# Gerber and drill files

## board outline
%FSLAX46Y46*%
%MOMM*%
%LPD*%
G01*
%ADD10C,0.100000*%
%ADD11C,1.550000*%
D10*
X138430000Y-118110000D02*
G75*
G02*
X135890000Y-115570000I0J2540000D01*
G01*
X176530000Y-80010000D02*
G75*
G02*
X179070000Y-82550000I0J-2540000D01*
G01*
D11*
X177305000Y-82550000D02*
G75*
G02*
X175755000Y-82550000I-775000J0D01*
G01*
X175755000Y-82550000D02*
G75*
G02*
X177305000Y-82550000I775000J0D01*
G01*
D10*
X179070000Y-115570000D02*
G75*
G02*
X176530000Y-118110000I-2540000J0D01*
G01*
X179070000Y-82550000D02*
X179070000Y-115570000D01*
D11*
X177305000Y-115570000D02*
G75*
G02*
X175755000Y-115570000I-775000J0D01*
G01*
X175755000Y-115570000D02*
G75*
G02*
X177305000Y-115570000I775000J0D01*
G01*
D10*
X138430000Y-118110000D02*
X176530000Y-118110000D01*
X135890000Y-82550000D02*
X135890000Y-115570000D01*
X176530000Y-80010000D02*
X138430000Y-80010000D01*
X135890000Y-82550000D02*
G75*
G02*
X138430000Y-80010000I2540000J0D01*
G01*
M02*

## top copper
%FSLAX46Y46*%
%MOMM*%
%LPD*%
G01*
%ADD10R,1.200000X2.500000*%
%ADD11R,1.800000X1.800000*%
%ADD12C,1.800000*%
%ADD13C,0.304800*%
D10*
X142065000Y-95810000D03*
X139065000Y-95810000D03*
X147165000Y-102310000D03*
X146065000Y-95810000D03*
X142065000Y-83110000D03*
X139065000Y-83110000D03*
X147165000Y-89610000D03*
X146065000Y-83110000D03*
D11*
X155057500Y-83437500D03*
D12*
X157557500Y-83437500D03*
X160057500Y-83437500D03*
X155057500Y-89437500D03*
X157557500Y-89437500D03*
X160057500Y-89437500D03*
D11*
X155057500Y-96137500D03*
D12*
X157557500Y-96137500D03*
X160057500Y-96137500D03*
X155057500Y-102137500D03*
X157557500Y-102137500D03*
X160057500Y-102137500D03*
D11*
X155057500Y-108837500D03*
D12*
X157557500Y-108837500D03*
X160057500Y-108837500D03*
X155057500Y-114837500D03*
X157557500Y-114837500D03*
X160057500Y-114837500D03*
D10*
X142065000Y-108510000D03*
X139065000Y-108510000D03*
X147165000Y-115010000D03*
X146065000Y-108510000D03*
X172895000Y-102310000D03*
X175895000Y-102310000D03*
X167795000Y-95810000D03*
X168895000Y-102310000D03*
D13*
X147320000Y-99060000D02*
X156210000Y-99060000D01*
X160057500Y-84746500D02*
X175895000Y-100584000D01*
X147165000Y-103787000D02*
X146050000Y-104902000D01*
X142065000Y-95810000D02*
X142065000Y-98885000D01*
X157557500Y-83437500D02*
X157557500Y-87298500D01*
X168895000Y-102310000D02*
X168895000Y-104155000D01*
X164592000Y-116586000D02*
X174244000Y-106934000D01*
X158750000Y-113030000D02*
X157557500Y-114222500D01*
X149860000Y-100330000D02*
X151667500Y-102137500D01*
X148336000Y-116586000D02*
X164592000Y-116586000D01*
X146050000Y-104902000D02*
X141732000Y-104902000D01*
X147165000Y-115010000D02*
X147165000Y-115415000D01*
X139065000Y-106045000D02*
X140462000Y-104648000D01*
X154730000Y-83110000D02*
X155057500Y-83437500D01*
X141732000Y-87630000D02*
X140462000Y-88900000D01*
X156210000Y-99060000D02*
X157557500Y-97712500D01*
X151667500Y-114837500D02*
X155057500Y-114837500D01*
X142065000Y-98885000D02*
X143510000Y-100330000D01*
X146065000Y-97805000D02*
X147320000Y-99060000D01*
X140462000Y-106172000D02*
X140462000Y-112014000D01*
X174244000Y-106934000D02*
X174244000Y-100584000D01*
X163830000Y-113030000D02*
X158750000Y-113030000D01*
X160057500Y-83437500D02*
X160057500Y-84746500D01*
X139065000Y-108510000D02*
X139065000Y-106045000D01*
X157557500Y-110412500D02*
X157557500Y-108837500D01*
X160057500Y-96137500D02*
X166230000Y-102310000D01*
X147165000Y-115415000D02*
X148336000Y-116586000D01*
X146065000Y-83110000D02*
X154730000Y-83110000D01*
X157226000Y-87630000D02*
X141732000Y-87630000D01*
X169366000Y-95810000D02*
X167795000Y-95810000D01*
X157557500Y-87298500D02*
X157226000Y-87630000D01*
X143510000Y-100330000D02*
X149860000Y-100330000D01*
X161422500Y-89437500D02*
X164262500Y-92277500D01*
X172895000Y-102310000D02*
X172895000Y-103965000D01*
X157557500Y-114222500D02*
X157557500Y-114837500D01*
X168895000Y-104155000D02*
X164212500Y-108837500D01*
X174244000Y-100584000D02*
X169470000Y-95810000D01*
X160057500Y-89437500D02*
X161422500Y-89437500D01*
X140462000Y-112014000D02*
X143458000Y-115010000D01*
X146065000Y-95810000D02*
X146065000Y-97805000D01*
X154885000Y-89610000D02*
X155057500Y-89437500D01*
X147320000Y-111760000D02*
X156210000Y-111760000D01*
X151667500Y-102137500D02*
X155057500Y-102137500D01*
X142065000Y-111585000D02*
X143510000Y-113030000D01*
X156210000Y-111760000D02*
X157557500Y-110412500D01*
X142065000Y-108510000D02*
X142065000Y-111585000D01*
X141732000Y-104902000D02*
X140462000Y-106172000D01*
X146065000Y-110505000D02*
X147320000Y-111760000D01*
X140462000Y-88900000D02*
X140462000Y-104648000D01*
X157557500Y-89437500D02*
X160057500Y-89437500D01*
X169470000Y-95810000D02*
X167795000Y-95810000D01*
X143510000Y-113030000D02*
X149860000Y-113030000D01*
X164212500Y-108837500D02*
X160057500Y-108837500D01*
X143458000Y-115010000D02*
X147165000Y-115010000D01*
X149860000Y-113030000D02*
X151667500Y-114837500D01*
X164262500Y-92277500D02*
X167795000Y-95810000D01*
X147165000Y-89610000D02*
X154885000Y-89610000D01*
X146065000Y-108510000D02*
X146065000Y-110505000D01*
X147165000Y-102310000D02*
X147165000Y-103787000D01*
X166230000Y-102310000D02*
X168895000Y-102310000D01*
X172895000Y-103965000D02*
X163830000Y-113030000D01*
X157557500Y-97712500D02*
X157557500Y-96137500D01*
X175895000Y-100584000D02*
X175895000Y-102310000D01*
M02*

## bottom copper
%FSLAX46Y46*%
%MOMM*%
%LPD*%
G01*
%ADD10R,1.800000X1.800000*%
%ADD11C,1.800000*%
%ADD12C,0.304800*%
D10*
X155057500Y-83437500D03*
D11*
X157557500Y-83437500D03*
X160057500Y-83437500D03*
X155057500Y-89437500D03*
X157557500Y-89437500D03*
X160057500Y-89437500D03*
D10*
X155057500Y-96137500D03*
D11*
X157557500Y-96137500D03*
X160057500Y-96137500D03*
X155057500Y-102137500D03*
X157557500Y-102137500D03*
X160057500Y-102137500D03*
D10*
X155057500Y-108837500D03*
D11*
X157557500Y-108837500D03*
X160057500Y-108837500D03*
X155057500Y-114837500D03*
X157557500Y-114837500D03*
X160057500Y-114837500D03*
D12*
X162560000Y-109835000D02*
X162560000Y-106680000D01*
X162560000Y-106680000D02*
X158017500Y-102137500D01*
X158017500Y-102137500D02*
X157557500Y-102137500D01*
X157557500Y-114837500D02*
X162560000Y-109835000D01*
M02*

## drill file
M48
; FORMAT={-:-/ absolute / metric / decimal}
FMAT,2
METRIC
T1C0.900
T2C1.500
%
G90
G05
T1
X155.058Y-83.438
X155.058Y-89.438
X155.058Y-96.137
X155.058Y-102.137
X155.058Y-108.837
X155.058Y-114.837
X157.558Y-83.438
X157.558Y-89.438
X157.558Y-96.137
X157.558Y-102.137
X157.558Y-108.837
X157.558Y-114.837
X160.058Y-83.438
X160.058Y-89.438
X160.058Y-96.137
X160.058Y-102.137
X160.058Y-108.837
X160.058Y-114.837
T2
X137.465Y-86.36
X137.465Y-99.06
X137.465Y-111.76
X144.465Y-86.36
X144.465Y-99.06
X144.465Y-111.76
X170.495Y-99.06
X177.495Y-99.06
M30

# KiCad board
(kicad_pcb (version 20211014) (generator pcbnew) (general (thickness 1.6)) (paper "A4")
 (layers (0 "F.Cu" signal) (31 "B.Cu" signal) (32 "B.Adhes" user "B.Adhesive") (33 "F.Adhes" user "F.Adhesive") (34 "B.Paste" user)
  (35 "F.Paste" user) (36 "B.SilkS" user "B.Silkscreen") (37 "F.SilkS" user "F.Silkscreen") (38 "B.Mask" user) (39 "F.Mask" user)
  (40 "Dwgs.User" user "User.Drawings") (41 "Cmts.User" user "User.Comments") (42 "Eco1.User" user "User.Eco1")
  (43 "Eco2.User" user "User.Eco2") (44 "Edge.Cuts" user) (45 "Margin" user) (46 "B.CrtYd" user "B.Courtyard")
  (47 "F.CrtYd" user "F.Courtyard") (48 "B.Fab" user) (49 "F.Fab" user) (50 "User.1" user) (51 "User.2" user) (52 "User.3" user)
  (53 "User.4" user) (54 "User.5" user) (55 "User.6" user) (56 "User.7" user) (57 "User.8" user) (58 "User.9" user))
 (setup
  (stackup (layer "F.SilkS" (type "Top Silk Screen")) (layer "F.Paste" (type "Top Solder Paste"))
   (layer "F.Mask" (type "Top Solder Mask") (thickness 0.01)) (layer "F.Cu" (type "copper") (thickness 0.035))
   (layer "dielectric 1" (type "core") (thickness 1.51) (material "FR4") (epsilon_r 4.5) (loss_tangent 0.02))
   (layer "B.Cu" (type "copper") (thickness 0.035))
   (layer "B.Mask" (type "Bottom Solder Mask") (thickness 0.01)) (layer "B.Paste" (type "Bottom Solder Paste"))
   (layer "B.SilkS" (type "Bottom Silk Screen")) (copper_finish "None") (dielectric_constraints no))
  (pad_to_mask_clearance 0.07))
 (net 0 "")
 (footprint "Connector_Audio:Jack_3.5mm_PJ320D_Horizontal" (layer "F.Cu") (at 142.24 99.06)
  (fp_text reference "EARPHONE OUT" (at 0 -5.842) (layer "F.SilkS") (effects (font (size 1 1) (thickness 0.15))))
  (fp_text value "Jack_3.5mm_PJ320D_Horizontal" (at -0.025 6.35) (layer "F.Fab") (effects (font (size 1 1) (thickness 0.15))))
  (pad "" np_thru_hole circle (at -4.775 0) (size 1.5 1.5) (drill 1.5) (layers *.Cu *.Mask))
  (pad "" np_thru_hole circle (at 2.225 0) (size 1.5 1.5) (drill 1.5) (layers *.Cu *.Mask))
  (pad "R1" smd rect (at -0.175 -3.25) (size 1.2 2.5) (layers "F.Cu" "F.Paste" "F.Mask"))
  (pad "R2" smd rect (at -3.175 -3.25) (size 1.2 2.5) (layers "F.Cu" "F.Paste" "F.Mask"))
  (pad "S" smd rect (at 4.925 3.25) (size 1.2 2.5) (layers "F.Cu" "F.Paste" "F.Mask"))
  (pad "T" smd rect (at 3.825 -3.25) (size 1.2 2.5) (layers "F.Cu" "F.Paste" "F.Mask")))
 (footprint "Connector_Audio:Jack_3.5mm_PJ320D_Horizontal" (layer "F.Cu") (at 142.24 86.36)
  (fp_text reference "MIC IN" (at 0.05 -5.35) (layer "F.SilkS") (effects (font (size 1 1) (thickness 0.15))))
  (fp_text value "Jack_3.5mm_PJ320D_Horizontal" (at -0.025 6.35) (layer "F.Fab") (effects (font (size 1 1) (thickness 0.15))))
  (pad "" np_thru_hole circle (at 2.225 0) (size 1.5 1.5) (drill 1.5) (layers *.Cu *.Mask))
  (pad "" np_thru_hole circle (at -4.775 0) (size 1.5 1.5) (drill 1.5) (layers *.Cu *.Mask))
  (pad "R1" smd rect (at -0.175 -3.25) (size 1.2 2.5) (layers "F.Cu" "F.Paste" "F.Mask"))
  (pad "R2" smd rect (at -3.175 -3.25) (size 1.2 2.5) (layers "F.Cu" "F.Paste" "F.Mask"))
  (pad "S" smd rect (at 4.925 3.25) (size 1.2 2.5) (layers "F.Cu" "F.Paste" "F.Mask"))
  (pad "T" smd rect (at 3.825 -3.25) (size 1.2 2.5) (layers "F.Cu" "F.Paste" "F.Mask")))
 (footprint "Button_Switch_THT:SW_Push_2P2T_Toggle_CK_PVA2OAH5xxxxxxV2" (layer "F.Cu") (at 155.0575 83.4375)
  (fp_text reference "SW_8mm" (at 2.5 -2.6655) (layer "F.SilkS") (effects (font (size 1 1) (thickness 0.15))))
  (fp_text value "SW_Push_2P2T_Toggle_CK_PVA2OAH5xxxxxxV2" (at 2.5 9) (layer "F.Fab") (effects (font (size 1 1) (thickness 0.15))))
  (pad "1" thru_hole rect (at 0 0) (size 1.8 1.8) (drill 0.9) (layers *.Cu *.Mask))
  (pad "2" thru_hole circle (at 2.5 0) (size 1.8 1.8) (drill 0.9) (layers *.Cu *.Mask))
  (pad "3" thru_hole circle (at 5 0) (size 1.8 1.8) (drill 0.9) (layers *.Cu *.Mask))
  (pad "4" thru_hole circle (at 0 6) (size 1.8 1.8) (drill 0.9) (layers *.Cu *.Mask))
  (pad "5" thru_hole circle (at 2.5 6) (size 1.8 1.8) (drill 0.9) (layers *.Cu *.Mask))
  (pad "6" thru_hole circle (at 5 6) (size 1.8 1.8) (drill 0.9) (layers *.Cu *.Mask)))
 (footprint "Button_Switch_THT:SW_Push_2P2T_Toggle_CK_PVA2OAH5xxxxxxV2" (layer "F.Cu") (at 155.0575 96.1375)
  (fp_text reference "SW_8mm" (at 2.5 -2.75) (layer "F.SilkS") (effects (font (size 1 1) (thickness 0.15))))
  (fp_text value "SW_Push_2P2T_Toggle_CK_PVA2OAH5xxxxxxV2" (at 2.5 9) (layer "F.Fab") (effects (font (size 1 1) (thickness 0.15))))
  (pad "1" thru_hole rect (at 0 0) (size 1.8 1.8) (drill 0.9) (layers *.Cu *.Mask))
  (pad "2" thru_hole circle (at 2.5 0) (size 1.8 1.8) (drill 0.9) (layers *.Cu *.Mask))
  (pad "3" thru_hole circle (at 5 0) (size 1.8 1.8) (drill 0.9) (layers *.Cu *.Mask))
  (pad "4" thru_hole circle (at 0 6) (size 1.8 1.8) (drill 0.9) (layers *.Cu *.Mask))
  (pad "5" thru_hole circle (at 2.5 6) (size 1.8 1.8) (drill 0.9) (layers *.Cu *.Mask))
  (pad "6" thru_hole circle (at 5 6) (size 1.8 1.8) (drill 0.9) (layers *.Cu *.Mask)))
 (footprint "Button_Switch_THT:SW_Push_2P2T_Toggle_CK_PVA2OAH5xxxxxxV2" (layer "F.Cu") (at 155.0575 108.8375)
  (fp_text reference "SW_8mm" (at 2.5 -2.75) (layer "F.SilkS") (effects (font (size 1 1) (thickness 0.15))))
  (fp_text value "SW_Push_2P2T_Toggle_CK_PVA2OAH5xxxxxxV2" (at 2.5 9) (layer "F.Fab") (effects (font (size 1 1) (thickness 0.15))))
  (pad "1" thru_hole rect (at 0 0) (size 1.8 1.8) (drill 0.9) (layers *.Cu *.Mask))
  (pad "2" thru_hole circle (at 2.5 0) (size 1.8 1.8) (drill 0.9) (layers *.Cu *.Mask))
  (pad "3" thru_hole circle (at 5 0) (size 1.8 1.8) (drill 0.9) (layers *.Cu *.Mask))
  (pad "4" thru_hole circle (at 0 6) (size 1.8 1.8) (drill 0.9) (layers *.Cu *.Mask))
  (pad "5" thru_hole circle (at 2.5 6) (size 1.8 1.8) (drill 0.9) (layers *.Cu *.Mask))
  (pad "6" thru_hole circle (at 5 6) (size 1.8 1.8) (drill 0.9) (layers *.Cu *.Mask)))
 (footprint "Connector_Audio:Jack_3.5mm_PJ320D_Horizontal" (layer "F.Cu") (at 142.24 111.76)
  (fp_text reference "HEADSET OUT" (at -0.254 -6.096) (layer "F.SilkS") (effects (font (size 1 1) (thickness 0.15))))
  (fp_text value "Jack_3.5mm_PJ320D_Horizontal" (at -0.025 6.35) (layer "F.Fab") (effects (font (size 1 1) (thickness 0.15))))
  (pad "" np_thru_hole circle (at -4.775 0) (size 1.5 1.5) (drill 1.5) (layers *.Cu *.Mask))
  (pad "" np_thru_hole circle (at 2.225 0) (size 1.5 1.5) (drill 1.5) (layers *.Cu *.Mask))
  (pad "R1" smd rect (at -0.175 -3.25) (size 1.2 2.5) (layers "F.Cu" "F.Paste" "F.Mask"))
  (pad "R2" smd rect (at -3.175 -3.25) (size 1.2 2.5) (layers "F.Cu" "F.Paste" "F.Mask"))
  (pad "S" smd rect (at 4.925 3.25) (size 1.2 2.5) (layers "F.Cu" "F.Paste" "F.Mask"))
  (pad "T" smd rect (at 3.825 -3.25) (size 1.2 2.5) (layers "F.Cu" "F.Paste" "F.Mask")))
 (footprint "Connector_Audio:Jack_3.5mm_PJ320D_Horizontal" (layer "F.Cu") (at 172.72 99.06 180)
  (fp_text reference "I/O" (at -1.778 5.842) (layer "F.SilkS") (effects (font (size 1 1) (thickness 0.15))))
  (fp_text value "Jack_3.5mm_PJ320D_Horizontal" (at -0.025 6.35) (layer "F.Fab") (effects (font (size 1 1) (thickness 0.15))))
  (pad "" np_thru_hole circle (at -4.775 0 180) (size 1.5 1.5) (drill 1.5) (layers *.Cu *.Mask))
  (pad "" np_thru_hole circle (at 2.225 0 180) (size 1.5 1.5) (drill 1.5) (layers *.Cu *.Mask))
  (pad "R1" smd rect (at -0.175 -3.25 180) (size 1.2 2.5) (layers "F.Cu" "F.Paste" "F.Mask"))
  (pad "R2" smd rect (at -3.175 -3.25 180) (size 1.2 2.5) (layers "F.Cu" "F.Paste" "F.Mask"))
  (pad "S" smd rect (at 4.925 3.25 180) (size 1.2 2.5) (layers "F.Cu" "F.Paste" "F.Mask"))
  (pad "T" smd rect (at 3.825 -3.25 180) (size 1.2 2.5) (layers "F.Cu" "F.Paste" "F.Mask")))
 (gr_arc (start 138.43 118.11) (mid 136.633949 117.366051) (end 135.89 115.57) (layer "Edge.Cuts") (width 0.1))
 (gr_arc (start 176.53 80.01) (mid 178.326051 80.753949) (end 179.07 82.55) (layer "Edge.Cuts") (width 0.1))
 (gr_circle (center 176.53 82.55) (end 178.03 82.55) (layer "Edge.Cuts") (width 0.1) (fill solid))
 (gr_arc (start 179.07 115.57) (mid 178.326051 117.366051) (end 176.53 118.11) (layer "Edge.Cuts") (width 0.1))
 (gr_line (start 179.07 82.55) (end 179.07 115.57) (layer "Edge.Cuts") (width 0.1))
 (gr_circle (center 176.53 115.57) (end 178.03 115.57) (layer "Edge.Cuts") (width 0.1) (fill solid))
 (gr_line (start 138.43 118.11) (end 176.53 118.11) (layer "Edge.Cuts") (width 0.1))
 (gr_line (start 135.89 82.55) (end 135.89 115.57) (layer "Edge.Cuts") (width 0.1))
 (gr_line (start 176.53 80.01) (end 138.43 80.01) (layer "Edge.Cuts") (width 0.1))
 (gr_arc (start 135.89 82.55) (mid 136.633949 80.753949) (end 138.43 80.01) (layer "Edge.Cuts") (width 0.1))
 (segment (start 147.32 99.06) (end 156.21 99.06) (width 0.3048) (layer "F.Cu") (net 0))
 (segment (start 160.0575 84.7465) (end 175.895 100.584) (width 0.3048) (layer "F.Cu") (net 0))
 (segment (start 147.165 103.787) (end 146.05 104.902) (width 0.3048) (layer "F.Cu") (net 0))
 (segment (start 142.065 95.81) (end 142.065 98.885) (width 0.3048) (layer "F.Cu") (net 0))
 (segment (start 157.5575 83.4375) (end 157.5575 87.2985) (width 0.3048) (layer "F.Cu") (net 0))
 (segment (start 168.895 102.31) (end 168.895 104.155) (width 0.3048) (layer "F.Cu") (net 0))
 (segment (start 164.592 116.586) (end 174.244 106.934) (width 0.3048) (layer "F.Cu") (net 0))
 (segment (start 158.75 113.03) (end 157.5575 114.2225) (width 0.3048) (layer "F.Cu") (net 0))
 (segment (start 149.86 100.33) (end 151.6675 102.1375) (width 0.3048) (layer "F.Cu") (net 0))
 (segment (start 148.336 116.586) (end 164.592 116.586) (width 0.3048) (layer "F.Cu") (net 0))
 (segment (start 146.05 104.902) (end 141.732 104.902) (width 0.3048) (layer "F.Cu") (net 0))
 (segment (start 147.165 115.01) (end 147.165 115.415) (width 0.3048) (layer "F.Cu") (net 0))
 (segment (start 139.065 106.045) (end 140.462 104.648) (width 0.3048) (layer "F.Cu") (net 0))
 (segment (start 154.73 83.11) (end 155.0575 83.4375) (width 0.3048) (layer "F.Cu") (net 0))
 (segment (start 141.732 87.63) (end 140.462 88.9) (width 0.3048) (layer "F.Cu") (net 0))
 (segment (start 156.21 99.06) (end 157.5575 97.7125) (width 0.3048) (layer "F.Cu") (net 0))
 (segment (start 151.6675 114.8375) (end 155.0575 114.8375) (width 0.3048) (layer "F.Cu") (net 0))
 (segment (start 142.065 98.885) (end 143.51 100.33) (width 0.3048) (layer "F.Cu") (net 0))
 (segment (start 146.065 97.805) (end 147.32 99.06) (width 0.3048) (layer "F.Cu") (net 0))
 (segment (start 140.462 106.172) (end 140.462 112.014) (width 0.3048) (layer "F.Cu") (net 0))
 (segment (start 174.244 106.934) (end 174.244 100.584) (width 0.3048) (layer "F.Cu") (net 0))
 (segment (start 163.83 113.03) (end 158.75 113.03) (width 0.3048) (layer "F.Cu") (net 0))
 (segment (start 160.0575 83.4375) (end 160.0575 84.7465) (width 0.3048) (layer "F.Cu") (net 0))
 (segment (start 139.065 108.51) (end 139.065 106.045) (width 0.3048) (layer "F.Cu") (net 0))
 (segment (start 157.5575 110.4125) (end 157.5575 108.8375) (width 0.3048) (layer "F.Cu") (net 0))
 (segment (start 160.0575 96.1375) (end 166.23 102.31) (width 0.3048) (layer "F.Cu") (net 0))
 (segment (start 147.165 115.415) (end 148.336 116.586) (width 0.3048) (layer "F.Cu") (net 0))
 (segment (start 146.065 83.11) (end 154.73 83.11) (width 0.3048) (layer "F.Cu") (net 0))
 (segment (start 157.226 87.63) (end 141.732 87.63) (width 0.3048) (layer "F.Cu") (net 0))
 (segment (start 169.366 95.81) (end 167.795 95.81) (width 0.3048) (layer "F.Cu") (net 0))
 (segment (start 157.5575 87.2985) (end 157.226 87.63) (width 0.3048) (layer "F.Cu") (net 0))
 (segment (start 143.51 100.33) (end 149.86 100.33) (width 0.3048) (layer "F.Cu") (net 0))
 (segment (start 161.4225 89.4375) (end 164.2625 92.2775) (width 0.3048) (layer "F.Cu") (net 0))
 (segment (start 172.895 102.31) (end 172.895 103.965) (width 0.3048) (layer "F.Cu") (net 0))
 (segment (start 157.5575 114.2225) (end 157.5575 114.8375) (width 0.3048) (layer "F.Cu") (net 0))
 (segment (start 168.895 104.155) (end 164.2125 108.8375) (width 0.3048) (layer "F.Cu") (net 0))
 (segment (start 174.244 100.584) (end 169.47 95.81) (width 0.3048) (layer "F.Cu") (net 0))
 (segment (start 160.0575 89.4375) (end 161.4225 89.4375) (width 0.3048) (layer "F.Cu") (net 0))
 (segment (start 140.462 112.014) (end 143.458 115.01) (width 0.3048) (layer "F.Cu") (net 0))
 (segment (start 146.065 95.81) (end 146.065 97.805) (width 0.3048) (layer "F.Cu") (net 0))
 (segment (start 154.885 89.61) (end 155.0575 89.4375) (width 0.3048) (layer "F.Cu") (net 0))
 (segment (start 147.32 111.76) (end 156.21 111.76) (width 0.3048) (layer "F.Cu") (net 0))
 (segment (start 151.6675 102.1375) (end 155.0575 102.1375) (width 0.3048) (layer "F.Cu") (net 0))
 (segment (start 142.065 111.585) (end 143.51 113.03) (width 0.3048) (layer "F.Cu") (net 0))
 (segment (start 156.21 111.76) (end 157.5575 110.4125) (width 0.3048) (layer "F.Cu") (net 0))
 (segment (start 142.065 108.51) (end 142.065 111.585) (width 0.3048) (layer "F.Cu") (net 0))
 (segment (start 141.732 104.902) (end 140.462 106.172) (width 0.3048) (layer "F.Cu") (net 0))
 (segment (start 146.065 110.505) (end 147.32 111.76) (width 0.3048) (layer "F.Cu") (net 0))
 (segment (start 140.462 88.9) (end 140.462 104.648) (width 0.3048) (layer "F.Cu") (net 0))
 (segment (start 157.5575 89.4375) (end 160.0575 89.4375) (width 0.3048) (layer "F.Cu") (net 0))
 (segment (start 169.47 95.81) (end 167.795 95.81) (width 0.3048) (layer "F.Cu") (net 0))
 (segment (start 143.51 113.03) (end 149.86 113.03) (width 0.3048) (layer "F.Cu") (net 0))
 (segment (start 164.2125 108.8375) (end 160.0575 108.8375) (width 0.3048) (layer "F.Cu") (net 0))
 (segment (start 143.458 115.01) (end 147.165 115.01) (width 0.3048) (layer "F.Cu") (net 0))
 (segment (start 149.86 113.03) (end 151.6675 114.8375) (width 0.3048) (layer "F.Cu") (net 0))
 (segment (start 164.2625 92.2775) (end 167.795 95.81) (width 0.3048) (layer "F.Cu") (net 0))
 (segment (start 147.165 89.61) (end 154.885 89.61) (width 0.3048) (layer "F.Cu") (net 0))
 (segment (start 146.065 108.51) (end 146.065 110.505) (width 0.3048) (layer "F.Cu") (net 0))
 (segment (start 147.165 102.31) (end 147.165 103.787) (width 0.3048) (layer "F.Cu") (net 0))
 (segment (start 166.23 102.31) (end 168.895 102.31) (width 0.3048) (layer "F.Cu") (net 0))
 (segment (start 172.895 103.965) (end 163.83 113.03) (width 0.3048) (layer "F.Cu") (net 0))
 (segment (start 157.5575 97.7125) (end 157.5575 96.1375) (width 0.3048) (layer "F.Cu") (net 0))
 (segment (start 175.895 100.584) (end 175.895 102.31) (width 0.3048) (layer "F.Cu") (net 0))
 (segment (start 162.56 109.835) (end 162.56 106.68) (width 0.3048) (layer "B.Cu") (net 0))
 (segment (start 162.56 106.68) (end 158.0175 102.1375) (width 0.3048) (layer "B.Cu") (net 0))
 (segment (start 158.0175 102.1375) (end 157.5575 102.1375) (width 0.3048) (layer "B.Cu") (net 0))
 (segment (start 157.5575 114.8375) (end 162.56 109.835) (width 0.3048) (layer "B.Cu") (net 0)))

